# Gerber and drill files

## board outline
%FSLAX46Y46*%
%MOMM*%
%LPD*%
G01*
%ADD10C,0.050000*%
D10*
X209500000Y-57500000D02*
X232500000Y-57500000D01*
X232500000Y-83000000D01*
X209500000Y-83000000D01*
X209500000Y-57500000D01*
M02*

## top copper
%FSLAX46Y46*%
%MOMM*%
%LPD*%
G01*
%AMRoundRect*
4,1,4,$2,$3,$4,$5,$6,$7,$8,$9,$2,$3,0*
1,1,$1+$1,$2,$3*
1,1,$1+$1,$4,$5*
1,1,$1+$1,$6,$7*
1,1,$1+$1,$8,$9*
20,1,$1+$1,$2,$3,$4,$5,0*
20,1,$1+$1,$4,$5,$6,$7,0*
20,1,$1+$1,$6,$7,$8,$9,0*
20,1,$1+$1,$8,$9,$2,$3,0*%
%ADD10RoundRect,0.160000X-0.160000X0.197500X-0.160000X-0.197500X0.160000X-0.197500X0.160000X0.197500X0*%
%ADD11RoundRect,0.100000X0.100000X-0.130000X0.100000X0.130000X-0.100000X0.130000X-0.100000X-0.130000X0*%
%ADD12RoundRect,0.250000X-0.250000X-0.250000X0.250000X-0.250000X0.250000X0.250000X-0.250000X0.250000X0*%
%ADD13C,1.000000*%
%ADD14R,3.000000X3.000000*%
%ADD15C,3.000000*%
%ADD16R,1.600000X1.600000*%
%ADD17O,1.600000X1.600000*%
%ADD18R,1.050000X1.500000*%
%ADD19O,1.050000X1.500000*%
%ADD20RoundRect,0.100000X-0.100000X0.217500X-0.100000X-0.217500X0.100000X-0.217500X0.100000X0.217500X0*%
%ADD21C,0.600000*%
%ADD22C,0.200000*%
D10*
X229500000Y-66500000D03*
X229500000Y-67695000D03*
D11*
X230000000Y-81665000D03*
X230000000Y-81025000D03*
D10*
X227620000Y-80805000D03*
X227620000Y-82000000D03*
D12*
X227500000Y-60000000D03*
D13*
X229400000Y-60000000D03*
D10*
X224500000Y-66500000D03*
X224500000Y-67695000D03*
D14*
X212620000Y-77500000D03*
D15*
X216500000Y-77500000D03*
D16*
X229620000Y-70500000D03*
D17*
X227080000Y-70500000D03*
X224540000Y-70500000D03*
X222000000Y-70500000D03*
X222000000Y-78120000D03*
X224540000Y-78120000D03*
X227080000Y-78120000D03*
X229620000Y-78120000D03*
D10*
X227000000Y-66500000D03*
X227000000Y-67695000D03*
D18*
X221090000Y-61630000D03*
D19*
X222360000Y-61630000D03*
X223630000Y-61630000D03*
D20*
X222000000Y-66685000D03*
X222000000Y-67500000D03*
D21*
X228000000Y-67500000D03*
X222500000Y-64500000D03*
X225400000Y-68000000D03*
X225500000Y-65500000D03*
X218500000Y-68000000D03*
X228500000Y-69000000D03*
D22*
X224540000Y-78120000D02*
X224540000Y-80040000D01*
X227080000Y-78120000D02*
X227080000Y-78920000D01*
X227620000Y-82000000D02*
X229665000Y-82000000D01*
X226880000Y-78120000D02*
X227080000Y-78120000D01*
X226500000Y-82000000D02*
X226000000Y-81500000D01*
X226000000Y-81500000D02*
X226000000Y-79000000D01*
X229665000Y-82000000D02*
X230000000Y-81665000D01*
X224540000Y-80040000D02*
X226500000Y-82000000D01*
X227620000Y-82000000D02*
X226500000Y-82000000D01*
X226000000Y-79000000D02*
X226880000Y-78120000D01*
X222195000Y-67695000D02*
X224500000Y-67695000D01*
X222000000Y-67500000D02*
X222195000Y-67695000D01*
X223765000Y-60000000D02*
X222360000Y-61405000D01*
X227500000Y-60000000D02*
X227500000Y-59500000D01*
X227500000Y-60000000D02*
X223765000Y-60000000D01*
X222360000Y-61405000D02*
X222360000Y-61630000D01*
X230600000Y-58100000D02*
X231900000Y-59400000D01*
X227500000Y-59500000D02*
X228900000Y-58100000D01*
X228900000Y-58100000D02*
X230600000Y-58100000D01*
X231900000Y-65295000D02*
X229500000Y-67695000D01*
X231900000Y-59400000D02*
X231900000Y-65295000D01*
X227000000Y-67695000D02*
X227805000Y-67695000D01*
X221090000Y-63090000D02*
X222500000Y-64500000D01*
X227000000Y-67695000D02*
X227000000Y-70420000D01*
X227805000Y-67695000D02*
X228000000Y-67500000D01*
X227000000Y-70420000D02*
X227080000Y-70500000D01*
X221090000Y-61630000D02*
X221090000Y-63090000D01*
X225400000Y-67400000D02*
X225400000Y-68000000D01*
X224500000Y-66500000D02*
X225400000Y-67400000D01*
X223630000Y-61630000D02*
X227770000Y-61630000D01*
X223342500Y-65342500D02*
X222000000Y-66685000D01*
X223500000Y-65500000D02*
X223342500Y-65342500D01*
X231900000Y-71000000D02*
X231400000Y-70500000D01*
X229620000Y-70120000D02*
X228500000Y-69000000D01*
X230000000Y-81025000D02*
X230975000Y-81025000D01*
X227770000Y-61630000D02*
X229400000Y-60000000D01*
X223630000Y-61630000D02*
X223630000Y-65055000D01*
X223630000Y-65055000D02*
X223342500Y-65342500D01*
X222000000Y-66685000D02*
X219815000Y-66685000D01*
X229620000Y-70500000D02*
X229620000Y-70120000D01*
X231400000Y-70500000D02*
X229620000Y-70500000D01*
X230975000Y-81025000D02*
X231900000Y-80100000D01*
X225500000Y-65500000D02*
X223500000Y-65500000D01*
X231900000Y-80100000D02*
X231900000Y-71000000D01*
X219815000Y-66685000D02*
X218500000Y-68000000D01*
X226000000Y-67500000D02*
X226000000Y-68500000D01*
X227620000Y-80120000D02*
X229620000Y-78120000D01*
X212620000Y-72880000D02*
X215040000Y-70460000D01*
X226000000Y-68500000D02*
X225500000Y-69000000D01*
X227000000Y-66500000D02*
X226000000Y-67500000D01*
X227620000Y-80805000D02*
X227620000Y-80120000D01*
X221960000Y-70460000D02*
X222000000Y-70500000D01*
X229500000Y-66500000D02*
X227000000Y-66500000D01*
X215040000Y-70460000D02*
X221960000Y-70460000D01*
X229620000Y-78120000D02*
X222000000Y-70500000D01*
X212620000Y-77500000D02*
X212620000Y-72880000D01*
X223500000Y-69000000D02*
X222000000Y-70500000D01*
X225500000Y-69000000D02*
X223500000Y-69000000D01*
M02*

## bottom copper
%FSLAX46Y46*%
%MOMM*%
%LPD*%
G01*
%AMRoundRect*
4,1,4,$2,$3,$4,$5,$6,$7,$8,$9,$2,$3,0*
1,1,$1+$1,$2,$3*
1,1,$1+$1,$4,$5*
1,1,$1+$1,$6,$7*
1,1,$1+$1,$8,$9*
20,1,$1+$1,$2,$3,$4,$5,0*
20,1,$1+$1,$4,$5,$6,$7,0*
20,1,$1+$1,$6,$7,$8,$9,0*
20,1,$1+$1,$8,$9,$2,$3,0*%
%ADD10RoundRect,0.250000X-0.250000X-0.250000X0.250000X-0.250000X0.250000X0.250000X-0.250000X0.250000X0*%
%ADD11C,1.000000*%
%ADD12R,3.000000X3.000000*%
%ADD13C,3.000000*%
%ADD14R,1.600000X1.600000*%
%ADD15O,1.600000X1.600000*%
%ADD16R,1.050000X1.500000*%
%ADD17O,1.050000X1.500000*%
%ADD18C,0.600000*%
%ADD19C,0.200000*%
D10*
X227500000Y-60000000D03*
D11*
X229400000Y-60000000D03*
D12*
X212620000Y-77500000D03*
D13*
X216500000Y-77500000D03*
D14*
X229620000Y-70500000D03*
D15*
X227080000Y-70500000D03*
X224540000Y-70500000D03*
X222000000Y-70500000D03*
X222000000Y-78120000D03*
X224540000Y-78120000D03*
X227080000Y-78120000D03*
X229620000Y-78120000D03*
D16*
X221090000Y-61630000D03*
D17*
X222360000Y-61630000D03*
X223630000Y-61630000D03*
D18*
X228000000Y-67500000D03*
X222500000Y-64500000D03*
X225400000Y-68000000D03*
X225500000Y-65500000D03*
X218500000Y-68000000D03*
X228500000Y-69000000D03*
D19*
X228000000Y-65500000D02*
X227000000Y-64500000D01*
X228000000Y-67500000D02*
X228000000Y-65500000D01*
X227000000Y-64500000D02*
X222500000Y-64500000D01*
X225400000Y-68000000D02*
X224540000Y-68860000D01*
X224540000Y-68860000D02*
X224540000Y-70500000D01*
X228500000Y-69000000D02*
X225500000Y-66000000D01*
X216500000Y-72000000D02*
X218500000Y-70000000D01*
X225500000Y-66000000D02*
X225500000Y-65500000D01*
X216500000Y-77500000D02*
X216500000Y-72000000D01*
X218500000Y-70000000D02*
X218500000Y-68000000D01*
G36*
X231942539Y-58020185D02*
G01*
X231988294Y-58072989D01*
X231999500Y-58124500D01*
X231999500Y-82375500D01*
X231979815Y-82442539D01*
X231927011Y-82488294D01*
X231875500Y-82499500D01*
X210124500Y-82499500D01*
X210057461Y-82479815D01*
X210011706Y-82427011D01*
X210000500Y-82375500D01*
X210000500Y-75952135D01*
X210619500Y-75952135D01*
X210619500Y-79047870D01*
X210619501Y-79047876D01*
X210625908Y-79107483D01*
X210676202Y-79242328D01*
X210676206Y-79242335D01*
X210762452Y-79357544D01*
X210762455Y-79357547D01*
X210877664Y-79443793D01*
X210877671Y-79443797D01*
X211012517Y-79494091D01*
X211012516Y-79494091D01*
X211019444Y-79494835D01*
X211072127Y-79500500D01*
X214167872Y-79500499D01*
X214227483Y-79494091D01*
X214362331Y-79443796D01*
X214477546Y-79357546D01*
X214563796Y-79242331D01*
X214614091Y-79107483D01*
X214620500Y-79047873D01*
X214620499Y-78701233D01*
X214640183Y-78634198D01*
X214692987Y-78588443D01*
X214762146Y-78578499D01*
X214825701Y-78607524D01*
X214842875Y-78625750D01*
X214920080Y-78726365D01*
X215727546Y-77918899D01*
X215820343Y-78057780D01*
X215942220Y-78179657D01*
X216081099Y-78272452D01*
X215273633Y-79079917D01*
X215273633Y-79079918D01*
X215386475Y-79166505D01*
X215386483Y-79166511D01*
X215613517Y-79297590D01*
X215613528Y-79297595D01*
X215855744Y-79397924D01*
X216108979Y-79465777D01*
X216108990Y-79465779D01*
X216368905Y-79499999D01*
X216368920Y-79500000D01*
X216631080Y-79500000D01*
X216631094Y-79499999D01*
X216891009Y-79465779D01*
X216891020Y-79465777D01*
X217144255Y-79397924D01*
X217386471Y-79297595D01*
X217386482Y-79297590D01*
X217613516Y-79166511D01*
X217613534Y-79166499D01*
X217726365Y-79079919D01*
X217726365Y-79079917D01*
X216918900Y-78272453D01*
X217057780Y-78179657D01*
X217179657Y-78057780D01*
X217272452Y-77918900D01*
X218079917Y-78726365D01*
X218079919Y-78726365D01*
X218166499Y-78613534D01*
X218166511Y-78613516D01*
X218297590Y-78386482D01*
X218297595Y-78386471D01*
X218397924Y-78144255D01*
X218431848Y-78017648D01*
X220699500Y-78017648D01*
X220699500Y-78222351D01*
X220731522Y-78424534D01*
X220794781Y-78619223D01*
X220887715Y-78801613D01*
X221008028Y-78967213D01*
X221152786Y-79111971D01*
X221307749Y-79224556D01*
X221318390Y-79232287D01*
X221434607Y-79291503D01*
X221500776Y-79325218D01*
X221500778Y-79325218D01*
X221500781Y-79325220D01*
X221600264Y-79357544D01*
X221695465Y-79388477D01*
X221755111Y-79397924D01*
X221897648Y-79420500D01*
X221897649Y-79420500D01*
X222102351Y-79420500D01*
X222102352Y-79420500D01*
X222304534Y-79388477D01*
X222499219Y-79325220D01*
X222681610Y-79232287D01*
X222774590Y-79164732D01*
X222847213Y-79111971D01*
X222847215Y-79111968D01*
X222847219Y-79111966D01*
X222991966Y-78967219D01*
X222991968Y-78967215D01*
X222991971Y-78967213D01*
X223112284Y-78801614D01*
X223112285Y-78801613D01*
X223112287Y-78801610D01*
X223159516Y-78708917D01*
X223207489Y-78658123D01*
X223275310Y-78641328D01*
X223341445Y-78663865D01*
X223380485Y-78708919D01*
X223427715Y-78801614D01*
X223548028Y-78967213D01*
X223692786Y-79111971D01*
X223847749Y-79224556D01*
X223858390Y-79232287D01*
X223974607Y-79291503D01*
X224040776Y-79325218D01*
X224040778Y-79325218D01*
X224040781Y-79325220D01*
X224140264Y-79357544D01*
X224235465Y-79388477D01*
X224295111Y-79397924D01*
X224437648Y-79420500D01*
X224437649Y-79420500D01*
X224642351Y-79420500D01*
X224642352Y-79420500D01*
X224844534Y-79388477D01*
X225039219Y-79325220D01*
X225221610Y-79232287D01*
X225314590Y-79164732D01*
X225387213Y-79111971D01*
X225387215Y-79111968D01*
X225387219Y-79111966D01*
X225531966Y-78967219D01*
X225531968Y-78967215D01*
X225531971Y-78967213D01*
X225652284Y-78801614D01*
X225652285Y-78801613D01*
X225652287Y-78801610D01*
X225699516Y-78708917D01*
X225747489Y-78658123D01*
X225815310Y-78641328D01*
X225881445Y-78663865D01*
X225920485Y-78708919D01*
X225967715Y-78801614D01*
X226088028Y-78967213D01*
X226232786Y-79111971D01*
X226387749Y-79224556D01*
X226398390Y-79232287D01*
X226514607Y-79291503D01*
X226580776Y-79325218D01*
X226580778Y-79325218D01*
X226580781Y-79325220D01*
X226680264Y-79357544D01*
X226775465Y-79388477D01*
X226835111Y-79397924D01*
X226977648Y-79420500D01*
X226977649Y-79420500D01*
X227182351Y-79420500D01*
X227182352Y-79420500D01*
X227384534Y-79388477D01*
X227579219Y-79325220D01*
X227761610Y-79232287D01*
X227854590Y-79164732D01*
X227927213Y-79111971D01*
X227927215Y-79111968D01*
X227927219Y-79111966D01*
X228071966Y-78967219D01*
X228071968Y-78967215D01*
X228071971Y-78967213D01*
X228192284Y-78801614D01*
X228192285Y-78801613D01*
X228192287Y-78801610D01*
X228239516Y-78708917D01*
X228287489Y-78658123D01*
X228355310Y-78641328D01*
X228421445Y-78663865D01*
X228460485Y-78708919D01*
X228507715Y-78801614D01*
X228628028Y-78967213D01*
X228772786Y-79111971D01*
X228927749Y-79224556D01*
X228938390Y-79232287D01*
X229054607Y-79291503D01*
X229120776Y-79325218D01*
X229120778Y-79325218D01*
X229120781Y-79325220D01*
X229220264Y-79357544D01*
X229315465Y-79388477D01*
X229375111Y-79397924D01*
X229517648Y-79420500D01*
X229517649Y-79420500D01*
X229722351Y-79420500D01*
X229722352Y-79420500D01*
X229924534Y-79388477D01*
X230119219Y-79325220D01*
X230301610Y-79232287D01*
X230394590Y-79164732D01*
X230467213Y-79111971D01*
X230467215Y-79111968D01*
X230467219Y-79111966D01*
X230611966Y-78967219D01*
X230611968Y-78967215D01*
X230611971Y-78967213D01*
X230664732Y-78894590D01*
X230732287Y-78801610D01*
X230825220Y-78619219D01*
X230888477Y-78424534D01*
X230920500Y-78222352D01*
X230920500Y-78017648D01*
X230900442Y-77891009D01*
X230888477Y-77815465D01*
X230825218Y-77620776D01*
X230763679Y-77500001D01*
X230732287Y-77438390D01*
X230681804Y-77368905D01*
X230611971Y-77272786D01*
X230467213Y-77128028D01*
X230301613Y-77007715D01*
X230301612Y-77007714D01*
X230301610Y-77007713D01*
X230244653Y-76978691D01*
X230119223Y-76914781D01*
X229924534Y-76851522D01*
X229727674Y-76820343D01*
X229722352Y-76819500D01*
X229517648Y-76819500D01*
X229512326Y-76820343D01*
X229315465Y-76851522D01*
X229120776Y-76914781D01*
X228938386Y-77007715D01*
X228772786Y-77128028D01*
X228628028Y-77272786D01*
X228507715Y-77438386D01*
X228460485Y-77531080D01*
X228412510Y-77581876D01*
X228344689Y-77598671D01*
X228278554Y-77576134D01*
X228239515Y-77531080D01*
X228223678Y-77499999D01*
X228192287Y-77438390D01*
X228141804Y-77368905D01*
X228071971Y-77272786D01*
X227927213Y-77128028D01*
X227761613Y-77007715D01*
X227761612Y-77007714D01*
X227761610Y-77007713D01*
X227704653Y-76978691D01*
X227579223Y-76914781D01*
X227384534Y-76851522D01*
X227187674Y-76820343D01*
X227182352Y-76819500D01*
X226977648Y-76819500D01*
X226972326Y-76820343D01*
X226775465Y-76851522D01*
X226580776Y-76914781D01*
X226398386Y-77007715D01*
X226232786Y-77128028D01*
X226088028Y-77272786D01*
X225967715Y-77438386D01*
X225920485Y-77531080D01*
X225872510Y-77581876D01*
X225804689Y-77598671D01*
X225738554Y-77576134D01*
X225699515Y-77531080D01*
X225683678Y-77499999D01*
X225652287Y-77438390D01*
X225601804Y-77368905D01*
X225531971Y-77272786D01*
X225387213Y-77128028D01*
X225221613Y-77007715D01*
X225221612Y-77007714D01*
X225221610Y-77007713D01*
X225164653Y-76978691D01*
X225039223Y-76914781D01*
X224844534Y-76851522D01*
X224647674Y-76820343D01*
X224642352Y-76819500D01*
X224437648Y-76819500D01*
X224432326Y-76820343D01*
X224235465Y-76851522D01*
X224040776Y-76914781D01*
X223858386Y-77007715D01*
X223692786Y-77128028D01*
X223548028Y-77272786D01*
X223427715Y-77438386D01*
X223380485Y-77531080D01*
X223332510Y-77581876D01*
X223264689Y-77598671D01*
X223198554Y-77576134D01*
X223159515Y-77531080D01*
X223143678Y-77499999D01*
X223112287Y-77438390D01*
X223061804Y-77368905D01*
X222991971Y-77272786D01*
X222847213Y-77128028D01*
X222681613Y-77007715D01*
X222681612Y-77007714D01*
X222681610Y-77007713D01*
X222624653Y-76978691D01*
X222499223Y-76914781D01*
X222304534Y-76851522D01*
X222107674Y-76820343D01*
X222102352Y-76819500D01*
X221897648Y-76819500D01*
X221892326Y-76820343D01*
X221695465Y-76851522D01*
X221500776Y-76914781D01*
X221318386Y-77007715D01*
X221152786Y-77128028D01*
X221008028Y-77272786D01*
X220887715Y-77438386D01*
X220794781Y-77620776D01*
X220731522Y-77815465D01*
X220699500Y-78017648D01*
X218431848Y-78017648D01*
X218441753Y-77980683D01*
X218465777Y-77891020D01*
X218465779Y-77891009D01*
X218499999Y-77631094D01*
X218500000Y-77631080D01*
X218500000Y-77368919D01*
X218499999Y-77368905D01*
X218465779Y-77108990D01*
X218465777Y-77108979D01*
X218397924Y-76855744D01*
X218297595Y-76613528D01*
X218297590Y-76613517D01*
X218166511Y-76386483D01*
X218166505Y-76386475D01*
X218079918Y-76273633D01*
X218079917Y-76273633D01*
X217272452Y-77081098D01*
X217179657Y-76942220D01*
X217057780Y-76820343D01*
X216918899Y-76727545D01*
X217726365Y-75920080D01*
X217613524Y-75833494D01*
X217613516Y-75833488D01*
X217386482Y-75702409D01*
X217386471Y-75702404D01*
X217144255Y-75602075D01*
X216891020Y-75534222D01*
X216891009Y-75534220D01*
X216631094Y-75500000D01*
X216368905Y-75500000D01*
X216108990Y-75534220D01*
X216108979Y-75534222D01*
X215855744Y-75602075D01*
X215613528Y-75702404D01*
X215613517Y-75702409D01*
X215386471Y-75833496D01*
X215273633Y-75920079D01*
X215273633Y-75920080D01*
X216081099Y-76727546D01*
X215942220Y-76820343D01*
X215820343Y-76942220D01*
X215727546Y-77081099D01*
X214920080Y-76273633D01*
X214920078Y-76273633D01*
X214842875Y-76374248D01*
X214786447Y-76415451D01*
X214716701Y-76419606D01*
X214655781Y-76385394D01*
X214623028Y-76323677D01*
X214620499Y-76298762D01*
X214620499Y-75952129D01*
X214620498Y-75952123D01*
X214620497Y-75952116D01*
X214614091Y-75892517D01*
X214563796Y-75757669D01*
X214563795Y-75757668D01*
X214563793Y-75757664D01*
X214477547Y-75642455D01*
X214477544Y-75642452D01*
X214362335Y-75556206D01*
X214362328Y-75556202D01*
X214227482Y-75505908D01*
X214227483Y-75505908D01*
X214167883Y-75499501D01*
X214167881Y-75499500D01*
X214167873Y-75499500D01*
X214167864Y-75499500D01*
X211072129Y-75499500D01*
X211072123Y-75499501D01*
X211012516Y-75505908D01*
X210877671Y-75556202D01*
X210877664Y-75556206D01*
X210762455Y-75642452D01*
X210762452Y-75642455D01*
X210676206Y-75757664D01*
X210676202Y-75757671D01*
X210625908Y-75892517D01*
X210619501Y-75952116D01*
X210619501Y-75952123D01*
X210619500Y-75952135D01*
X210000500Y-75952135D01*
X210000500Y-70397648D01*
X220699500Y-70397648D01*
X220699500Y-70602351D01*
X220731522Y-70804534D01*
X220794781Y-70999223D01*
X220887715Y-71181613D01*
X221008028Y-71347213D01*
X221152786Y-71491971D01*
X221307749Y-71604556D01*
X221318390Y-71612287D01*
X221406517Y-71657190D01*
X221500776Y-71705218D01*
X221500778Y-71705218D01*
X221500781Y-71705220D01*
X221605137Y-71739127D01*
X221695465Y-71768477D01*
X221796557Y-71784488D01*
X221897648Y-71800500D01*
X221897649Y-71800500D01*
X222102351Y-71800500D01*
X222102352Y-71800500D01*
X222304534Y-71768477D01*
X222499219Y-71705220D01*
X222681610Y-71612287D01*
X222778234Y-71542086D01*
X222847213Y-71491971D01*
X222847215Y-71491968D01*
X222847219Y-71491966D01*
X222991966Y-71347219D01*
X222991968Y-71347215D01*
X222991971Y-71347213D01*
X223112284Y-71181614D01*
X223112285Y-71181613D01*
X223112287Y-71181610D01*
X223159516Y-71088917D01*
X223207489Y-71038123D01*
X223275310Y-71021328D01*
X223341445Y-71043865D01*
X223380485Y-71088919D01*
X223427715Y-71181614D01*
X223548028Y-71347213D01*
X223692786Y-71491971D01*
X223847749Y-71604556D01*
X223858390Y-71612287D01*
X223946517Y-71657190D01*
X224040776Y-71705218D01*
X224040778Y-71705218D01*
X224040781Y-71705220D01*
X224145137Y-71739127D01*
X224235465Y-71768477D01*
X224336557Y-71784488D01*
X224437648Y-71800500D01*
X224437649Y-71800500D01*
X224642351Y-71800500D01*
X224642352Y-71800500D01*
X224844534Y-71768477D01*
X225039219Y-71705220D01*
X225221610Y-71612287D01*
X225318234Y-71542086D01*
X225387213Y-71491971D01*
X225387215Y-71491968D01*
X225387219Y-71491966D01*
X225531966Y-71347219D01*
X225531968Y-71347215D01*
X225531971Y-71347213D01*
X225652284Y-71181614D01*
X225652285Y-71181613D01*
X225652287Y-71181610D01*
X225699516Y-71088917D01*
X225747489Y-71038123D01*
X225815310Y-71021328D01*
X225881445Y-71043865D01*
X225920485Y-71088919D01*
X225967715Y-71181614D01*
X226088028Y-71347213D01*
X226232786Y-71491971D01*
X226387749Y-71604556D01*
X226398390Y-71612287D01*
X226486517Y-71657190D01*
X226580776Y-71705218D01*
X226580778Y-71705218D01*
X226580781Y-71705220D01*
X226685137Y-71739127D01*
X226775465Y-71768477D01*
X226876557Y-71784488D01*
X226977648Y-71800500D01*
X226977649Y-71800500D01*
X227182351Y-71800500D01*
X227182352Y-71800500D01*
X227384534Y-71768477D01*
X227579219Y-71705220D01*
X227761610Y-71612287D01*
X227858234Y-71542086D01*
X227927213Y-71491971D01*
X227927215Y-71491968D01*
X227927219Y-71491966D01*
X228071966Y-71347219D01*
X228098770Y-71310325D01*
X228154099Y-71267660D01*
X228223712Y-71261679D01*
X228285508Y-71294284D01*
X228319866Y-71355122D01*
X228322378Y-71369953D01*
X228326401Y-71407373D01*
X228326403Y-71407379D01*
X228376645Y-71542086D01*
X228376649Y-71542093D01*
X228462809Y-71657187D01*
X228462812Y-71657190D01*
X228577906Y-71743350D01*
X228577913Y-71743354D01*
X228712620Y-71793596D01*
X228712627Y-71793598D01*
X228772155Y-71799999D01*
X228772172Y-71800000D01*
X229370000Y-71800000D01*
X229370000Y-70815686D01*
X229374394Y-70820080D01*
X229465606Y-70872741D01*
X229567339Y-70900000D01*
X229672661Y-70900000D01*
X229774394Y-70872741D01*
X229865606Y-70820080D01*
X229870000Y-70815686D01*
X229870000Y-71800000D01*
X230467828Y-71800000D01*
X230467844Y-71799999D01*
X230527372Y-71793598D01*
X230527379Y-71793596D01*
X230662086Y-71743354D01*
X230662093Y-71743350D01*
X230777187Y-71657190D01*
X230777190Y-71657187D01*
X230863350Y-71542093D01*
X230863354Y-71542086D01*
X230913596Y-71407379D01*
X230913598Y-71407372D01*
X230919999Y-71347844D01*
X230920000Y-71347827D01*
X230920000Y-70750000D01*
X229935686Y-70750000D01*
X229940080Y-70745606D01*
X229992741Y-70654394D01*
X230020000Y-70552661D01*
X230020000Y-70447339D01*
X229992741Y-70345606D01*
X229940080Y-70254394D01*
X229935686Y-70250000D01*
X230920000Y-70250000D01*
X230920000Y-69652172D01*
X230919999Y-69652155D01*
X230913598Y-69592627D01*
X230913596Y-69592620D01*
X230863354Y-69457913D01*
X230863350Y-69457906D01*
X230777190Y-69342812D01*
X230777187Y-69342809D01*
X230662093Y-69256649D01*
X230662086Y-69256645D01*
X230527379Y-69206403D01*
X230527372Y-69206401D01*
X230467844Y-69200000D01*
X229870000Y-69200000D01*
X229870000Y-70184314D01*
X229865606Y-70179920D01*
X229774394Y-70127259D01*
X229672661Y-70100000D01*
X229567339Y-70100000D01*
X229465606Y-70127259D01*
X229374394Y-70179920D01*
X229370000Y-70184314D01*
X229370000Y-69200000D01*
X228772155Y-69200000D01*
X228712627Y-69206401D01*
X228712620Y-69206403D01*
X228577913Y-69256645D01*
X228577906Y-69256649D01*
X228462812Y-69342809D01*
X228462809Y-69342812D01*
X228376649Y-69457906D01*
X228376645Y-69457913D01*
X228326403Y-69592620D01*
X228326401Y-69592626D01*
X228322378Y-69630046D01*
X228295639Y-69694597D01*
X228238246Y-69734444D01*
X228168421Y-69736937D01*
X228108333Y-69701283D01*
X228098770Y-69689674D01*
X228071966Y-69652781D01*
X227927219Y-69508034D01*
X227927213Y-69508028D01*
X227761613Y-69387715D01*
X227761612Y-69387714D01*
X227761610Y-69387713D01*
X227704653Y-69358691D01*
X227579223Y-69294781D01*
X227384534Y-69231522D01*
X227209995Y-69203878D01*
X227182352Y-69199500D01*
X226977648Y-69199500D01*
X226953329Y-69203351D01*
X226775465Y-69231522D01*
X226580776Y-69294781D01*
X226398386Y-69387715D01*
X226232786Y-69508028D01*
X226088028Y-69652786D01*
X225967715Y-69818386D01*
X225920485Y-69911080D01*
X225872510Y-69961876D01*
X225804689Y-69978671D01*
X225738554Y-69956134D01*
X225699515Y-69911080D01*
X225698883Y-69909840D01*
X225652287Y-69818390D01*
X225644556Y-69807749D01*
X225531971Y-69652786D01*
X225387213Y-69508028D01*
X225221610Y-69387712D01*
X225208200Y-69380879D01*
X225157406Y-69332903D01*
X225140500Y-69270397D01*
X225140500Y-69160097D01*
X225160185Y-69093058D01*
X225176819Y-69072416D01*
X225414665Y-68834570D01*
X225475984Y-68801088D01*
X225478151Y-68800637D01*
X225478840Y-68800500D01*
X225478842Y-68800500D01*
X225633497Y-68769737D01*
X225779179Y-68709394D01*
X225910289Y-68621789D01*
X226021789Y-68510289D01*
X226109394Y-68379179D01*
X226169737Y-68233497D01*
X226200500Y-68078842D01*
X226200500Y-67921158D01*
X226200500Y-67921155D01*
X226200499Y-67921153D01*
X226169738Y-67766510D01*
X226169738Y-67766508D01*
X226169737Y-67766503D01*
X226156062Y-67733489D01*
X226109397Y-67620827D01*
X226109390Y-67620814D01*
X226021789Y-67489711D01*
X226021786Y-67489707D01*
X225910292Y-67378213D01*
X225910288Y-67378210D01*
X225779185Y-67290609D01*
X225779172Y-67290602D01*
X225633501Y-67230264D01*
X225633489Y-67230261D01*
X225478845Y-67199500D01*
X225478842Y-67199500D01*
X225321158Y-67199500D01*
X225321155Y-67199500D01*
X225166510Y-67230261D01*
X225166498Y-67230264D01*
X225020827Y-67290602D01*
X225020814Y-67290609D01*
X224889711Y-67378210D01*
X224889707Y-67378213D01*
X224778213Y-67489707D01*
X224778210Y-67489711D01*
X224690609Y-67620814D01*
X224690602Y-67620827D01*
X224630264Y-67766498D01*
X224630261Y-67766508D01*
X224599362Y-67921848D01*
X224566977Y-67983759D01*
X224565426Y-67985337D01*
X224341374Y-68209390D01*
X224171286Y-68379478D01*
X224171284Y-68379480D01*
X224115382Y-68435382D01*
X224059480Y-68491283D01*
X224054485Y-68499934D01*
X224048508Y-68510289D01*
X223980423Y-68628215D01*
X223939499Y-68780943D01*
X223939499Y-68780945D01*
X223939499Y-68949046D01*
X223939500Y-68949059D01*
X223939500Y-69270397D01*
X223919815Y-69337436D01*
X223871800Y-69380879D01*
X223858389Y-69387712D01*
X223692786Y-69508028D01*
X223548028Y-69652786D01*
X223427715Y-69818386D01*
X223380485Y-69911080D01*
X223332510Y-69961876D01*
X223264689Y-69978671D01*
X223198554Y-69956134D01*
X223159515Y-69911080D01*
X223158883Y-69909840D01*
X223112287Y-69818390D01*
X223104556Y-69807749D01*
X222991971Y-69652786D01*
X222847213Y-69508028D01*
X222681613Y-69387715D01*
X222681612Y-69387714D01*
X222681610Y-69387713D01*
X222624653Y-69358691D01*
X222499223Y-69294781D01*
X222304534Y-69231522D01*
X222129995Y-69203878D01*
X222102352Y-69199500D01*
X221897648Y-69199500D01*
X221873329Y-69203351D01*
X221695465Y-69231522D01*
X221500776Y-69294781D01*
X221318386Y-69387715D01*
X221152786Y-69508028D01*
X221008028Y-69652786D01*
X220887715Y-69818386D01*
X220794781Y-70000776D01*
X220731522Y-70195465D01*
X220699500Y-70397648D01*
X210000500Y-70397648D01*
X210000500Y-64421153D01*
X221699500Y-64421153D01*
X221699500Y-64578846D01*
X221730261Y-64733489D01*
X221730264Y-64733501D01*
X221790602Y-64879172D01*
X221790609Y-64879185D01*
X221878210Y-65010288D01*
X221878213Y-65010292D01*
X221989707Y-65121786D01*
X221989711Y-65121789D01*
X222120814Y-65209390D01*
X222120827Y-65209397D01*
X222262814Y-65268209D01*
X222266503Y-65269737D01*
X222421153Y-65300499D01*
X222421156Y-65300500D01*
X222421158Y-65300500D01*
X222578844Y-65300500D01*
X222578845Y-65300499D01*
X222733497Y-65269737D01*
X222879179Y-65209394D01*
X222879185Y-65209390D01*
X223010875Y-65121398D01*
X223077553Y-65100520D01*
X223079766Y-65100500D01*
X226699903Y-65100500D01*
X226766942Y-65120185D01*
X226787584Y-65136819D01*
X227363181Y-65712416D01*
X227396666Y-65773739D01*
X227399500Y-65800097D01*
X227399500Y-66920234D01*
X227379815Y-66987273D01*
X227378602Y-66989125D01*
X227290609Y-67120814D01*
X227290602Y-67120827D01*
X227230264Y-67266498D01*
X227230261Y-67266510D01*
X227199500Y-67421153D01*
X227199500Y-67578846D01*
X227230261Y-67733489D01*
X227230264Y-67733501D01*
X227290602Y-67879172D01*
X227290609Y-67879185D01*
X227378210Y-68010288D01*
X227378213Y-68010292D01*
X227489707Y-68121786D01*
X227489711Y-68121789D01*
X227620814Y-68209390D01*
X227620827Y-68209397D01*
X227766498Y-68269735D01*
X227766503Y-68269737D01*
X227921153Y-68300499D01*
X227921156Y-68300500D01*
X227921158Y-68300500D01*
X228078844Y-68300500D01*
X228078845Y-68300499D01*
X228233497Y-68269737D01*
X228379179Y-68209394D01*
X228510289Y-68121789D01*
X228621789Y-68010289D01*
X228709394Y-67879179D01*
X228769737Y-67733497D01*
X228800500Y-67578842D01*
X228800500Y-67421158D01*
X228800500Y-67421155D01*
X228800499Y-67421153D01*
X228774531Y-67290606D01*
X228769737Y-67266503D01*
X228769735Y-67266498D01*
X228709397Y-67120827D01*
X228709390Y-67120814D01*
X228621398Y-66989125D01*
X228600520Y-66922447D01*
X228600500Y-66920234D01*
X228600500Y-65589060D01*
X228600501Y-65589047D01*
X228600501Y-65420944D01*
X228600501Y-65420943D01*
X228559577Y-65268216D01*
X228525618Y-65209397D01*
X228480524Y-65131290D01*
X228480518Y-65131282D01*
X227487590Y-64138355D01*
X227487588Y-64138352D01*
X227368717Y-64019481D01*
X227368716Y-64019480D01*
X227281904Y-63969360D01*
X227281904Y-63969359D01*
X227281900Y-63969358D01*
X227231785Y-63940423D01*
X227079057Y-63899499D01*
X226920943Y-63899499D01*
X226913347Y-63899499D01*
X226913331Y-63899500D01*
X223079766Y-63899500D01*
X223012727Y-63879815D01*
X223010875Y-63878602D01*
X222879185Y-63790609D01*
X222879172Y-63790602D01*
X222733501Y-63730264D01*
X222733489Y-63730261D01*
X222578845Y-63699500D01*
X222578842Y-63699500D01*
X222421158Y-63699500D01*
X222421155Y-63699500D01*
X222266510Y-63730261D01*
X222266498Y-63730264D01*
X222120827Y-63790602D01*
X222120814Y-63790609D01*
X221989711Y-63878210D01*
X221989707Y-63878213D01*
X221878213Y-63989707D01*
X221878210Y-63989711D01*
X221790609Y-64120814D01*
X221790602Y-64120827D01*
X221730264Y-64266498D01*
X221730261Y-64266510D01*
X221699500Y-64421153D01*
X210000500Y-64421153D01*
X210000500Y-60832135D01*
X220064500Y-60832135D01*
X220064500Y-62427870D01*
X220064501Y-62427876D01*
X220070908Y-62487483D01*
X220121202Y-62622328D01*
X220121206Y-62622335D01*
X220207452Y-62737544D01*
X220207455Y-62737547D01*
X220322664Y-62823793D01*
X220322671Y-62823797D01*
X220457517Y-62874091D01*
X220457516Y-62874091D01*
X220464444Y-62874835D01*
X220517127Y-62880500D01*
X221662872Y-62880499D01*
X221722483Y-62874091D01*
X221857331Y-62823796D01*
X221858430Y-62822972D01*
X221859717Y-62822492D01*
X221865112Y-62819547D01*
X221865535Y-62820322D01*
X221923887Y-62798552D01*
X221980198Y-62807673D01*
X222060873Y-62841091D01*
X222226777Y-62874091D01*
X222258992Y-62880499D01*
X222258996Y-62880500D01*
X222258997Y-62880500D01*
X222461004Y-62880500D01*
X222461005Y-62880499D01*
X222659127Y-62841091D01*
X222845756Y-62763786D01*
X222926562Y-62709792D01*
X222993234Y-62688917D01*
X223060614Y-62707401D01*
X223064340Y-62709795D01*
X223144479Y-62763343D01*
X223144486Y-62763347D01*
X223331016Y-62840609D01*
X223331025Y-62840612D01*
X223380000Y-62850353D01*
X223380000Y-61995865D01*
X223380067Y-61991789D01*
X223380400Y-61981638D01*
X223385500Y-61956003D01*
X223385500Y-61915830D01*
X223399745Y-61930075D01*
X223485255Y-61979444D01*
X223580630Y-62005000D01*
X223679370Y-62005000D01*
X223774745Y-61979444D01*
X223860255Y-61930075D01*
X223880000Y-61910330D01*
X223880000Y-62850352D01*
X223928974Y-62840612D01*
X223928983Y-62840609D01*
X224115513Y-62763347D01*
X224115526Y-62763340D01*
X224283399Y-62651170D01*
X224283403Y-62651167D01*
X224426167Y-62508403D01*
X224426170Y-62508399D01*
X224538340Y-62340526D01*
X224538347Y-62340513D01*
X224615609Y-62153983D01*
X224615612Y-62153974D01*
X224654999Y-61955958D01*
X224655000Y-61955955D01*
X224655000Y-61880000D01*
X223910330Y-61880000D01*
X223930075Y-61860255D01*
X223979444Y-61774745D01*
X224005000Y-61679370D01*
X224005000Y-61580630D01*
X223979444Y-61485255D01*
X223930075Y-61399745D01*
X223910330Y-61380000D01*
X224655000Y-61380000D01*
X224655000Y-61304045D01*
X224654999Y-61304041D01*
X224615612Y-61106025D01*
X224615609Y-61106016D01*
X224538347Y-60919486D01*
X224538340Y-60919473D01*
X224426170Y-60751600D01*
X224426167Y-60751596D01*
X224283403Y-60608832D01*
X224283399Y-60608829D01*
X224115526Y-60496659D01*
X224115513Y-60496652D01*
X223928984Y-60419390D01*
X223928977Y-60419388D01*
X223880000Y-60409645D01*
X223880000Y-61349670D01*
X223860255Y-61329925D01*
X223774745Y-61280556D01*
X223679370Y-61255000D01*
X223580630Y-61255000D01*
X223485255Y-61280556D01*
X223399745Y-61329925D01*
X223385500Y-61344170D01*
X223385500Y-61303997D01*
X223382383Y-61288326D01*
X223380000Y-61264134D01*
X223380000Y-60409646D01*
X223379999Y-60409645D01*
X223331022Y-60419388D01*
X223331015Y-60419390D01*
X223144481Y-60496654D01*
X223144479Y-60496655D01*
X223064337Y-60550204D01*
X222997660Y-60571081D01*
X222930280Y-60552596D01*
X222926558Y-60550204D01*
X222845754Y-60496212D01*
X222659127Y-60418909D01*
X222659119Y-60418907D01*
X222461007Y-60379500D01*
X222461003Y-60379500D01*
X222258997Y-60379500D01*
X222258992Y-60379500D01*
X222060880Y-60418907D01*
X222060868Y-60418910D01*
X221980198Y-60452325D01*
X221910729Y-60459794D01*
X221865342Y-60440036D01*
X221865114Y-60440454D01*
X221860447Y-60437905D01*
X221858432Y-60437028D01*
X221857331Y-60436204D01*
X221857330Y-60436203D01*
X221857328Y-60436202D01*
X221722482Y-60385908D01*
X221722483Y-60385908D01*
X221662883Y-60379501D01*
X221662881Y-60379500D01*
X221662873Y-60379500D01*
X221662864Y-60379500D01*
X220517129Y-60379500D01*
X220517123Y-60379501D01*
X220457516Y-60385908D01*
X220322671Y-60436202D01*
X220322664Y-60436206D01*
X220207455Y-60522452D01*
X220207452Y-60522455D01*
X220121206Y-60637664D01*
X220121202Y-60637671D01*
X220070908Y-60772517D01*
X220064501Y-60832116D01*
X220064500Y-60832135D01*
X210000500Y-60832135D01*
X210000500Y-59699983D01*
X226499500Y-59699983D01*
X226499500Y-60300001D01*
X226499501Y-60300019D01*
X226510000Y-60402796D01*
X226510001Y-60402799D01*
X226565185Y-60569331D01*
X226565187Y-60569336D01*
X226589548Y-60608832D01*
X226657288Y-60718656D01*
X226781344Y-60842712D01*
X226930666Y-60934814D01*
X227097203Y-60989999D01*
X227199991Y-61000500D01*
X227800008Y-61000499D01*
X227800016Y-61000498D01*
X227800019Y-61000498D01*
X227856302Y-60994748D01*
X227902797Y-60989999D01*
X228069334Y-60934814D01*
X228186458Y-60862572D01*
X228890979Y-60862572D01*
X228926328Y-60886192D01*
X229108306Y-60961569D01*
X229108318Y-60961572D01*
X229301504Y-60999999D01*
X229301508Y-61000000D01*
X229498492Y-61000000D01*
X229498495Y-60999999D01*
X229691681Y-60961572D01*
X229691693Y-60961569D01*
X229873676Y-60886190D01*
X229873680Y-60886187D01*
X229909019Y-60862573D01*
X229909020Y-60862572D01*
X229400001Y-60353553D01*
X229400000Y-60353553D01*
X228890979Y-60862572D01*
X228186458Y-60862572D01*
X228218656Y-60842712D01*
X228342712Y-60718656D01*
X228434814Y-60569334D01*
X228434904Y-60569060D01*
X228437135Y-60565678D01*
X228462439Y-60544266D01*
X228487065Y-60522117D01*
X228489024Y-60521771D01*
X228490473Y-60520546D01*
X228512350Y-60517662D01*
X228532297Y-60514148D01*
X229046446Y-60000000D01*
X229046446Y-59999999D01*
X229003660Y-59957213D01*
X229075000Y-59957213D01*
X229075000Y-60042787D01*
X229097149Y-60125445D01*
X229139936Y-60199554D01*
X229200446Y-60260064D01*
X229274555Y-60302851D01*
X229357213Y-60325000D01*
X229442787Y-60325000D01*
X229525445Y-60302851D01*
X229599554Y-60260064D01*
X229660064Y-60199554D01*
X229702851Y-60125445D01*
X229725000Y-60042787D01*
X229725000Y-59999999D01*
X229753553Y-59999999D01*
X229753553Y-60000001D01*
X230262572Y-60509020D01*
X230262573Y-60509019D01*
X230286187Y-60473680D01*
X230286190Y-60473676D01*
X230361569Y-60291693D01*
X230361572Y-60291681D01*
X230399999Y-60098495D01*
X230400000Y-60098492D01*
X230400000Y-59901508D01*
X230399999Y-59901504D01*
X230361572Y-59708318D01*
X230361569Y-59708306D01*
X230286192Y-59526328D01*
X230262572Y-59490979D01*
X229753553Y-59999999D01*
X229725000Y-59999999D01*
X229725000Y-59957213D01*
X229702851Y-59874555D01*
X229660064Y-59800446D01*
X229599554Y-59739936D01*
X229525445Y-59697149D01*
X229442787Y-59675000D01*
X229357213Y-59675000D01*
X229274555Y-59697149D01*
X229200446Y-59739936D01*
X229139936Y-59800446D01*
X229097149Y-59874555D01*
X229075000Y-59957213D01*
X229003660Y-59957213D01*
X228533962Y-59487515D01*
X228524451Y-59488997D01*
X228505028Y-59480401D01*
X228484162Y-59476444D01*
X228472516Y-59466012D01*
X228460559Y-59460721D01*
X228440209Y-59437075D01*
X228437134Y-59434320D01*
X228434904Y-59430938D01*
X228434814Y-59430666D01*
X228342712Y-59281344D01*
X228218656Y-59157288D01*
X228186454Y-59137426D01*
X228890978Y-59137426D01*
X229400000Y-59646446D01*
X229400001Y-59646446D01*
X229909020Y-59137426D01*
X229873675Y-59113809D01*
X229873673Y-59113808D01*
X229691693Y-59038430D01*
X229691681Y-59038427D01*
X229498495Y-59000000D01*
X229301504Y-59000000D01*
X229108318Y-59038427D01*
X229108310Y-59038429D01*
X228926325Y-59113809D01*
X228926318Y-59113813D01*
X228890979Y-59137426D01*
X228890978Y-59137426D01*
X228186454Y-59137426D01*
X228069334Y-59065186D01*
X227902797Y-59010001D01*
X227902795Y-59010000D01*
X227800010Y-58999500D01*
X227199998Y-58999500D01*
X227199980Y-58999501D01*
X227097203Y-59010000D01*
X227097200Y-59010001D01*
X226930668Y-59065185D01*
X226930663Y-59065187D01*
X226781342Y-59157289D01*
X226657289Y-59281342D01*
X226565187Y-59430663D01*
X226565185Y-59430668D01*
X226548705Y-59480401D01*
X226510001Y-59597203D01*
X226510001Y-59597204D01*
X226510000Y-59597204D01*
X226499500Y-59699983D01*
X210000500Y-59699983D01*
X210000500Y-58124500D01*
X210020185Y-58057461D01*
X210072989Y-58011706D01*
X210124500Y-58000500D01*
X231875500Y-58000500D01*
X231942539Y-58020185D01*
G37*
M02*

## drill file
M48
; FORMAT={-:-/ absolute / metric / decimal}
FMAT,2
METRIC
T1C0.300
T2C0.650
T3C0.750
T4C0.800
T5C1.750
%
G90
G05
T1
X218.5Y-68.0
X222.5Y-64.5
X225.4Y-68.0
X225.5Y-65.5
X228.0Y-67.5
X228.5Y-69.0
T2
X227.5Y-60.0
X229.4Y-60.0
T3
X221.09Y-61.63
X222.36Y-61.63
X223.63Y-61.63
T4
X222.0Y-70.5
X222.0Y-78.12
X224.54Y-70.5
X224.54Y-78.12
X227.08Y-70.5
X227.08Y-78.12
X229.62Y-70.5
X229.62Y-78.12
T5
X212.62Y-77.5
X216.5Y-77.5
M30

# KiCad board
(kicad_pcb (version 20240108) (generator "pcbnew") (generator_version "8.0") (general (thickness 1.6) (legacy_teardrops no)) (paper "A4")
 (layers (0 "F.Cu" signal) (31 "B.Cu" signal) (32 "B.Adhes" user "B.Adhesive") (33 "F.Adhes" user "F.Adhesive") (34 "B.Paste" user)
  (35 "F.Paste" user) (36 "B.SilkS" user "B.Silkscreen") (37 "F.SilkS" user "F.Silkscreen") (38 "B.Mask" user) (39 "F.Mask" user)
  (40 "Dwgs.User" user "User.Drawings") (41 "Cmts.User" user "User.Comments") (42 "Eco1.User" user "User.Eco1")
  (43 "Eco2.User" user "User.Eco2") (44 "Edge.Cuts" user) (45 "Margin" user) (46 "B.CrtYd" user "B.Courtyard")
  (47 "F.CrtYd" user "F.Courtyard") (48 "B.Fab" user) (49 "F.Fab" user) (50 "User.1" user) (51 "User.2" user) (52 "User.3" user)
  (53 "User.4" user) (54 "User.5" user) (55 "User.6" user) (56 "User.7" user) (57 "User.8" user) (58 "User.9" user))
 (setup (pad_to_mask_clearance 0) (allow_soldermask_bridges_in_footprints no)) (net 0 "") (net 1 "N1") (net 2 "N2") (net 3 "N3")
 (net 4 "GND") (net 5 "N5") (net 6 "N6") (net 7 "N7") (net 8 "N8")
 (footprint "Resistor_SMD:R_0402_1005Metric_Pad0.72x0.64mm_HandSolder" (layer "F.Cu") (at 229.5 67.0975 -90)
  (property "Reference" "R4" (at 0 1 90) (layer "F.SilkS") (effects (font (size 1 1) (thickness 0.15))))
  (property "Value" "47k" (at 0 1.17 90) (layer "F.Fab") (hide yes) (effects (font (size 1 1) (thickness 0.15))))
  (pad "1" smd roundrect (at -0.5975 0 270) (size 0.715 0.64) (layers "F.Cu" "F.Paste" "F.Mask") (roundrect_rratio 0.25) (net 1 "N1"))
  (pad "2" smd roundrect (at 0.5975 0 270) (size 0.715 0.64) (layers "F.Cu" "F.Paste" "F.Mask") (roundrect_rratio 0.25) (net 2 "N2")))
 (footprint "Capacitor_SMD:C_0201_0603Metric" (layer "F.Cu") (at 230 81.345 90)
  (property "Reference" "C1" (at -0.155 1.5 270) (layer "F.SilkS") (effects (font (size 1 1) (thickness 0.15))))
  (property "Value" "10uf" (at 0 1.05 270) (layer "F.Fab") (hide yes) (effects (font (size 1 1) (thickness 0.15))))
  (pad "" smd roundrect (at -0.345 0 90) (size 0.318 0.36) (layers "F.Paste") (roundrect_rratio 0.25))
  (pad "" smd roundrect (at 0.345 0 90) (size 0.318 0.36) (layers "F.Paste") (roundrect_rratio 0.25))
  (pad "1" smd roundrect (at -0.32 0 90) (size 0.46 0.4) (layers "F.Cu" "F.Mask") (roundrect_rratio 0.25) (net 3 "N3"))
  (pad "2" smd roundrect (at 0.32 0 90) (size 0.46 0.4) (layers "F.Cu" "F.Mask") (roundrect_rratio 0.25) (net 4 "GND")))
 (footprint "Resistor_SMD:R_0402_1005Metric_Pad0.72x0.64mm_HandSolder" (layer "F.Cu") (at 227.62 81.4025 -90)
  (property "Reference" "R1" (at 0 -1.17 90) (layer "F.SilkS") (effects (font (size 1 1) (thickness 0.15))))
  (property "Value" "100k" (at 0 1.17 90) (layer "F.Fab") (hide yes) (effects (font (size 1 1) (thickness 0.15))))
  (pad "1" smd roundrect (at -0.5975 0 270) (size 0.715 0.64) (layers "F.Cu" "F.Paste" "F.Mask") (roundrect_rratio 0.25) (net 1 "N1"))
  (pad "2" smd roundrect (at 0.5975 0 270) (size 0.715 0.64) (layers "F.Cu" "F.Paste" "F.Mask") (roundrect_rratio 0.25) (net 3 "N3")))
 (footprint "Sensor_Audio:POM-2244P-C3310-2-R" (layer "F.Cu") (at 227.5 60)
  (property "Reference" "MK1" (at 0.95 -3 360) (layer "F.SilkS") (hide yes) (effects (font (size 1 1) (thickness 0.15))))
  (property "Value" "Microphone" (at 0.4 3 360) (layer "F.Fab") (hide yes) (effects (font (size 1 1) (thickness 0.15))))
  (pad "1" thru_hole roundrect (at 0 0) (size 1 1) (drill 0.65) (layers "*.Cu" "*.Mask") (remove_unused_layers no) (roundrect_rratio 0.25)
   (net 2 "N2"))
  (pad "2" thru_hole circle (at 1.9 0) (size 1 1) (drill 0.65) (layers "*.Cu" "*.Mask") (remove_unused_layers no) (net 4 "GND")))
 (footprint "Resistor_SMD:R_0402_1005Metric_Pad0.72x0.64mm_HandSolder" (layer "F.Cu") (at 224.5 67.0975 -90)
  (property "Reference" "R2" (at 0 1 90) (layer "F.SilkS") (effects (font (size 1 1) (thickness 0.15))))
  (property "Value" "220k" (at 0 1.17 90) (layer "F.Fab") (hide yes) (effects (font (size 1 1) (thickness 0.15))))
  (pad "1" smd roundrect (at -0.5975 0 270) (size 0.715 0.64) (layers "F.Cu" "F.Paste" "F.Mask") (roundrect_rratio 0.25) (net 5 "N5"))
  (pad "2" smd roundrect (at 0.5975 0 270) (size 0.715 0.64) (layers "F.Cu" "F.Paste" "F.Mask") (roundrect_rratio 0.25) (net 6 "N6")))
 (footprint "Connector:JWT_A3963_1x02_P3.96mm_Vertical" (layer "F.Cu") (at 212.62 77.5)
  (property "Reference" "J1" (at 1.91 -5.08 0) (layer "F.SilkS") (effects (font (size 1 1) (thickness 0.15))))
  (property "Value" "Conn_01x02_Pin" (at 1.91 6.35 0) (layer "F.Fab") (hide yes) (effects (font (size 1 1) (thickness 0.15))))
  (pad "1" thru_hole rect (at 0 0) (size 3 3) (drill 1.75) (layers "*.Cu" "*.Mask") (remove_unused_layers no) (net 1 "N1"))
  (pad "2" thru_hole circle (at 3.88 0) (size 3 3) (drill 1.75) (layers "*.Cu" "*.Mask") (remove_unused_layers no) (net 4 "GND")))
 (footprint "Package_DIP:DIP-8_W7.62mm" (layer "F.Cu") (at 229.62 70.5 -90)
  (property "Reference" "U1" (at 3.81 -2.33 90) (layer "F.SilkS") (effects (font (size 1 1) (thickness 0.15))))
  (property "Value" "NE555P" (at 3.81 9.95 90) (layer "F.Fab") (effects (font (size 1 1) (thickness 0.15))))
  (pad "1" thru_hole rect (at 0 0 270) (size 1.6 1.6) (drill 0.8) (layers "*.Cu" "*.Mask") (remove_unused_layers no) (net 4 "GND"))
  (pad "2" thru_hole oval (at 0 2.54 270) (size 1.6 1.6) (drill 0.8) (layers "*.Cu" "*.Mask") (remove_unused_layers no) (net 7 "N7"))
  (pad "3" thru_hole oval (at 0 5.08 270) (size 1.6 1.6) (drill 0.8) (layers "*.Cu" "*.Mask") (remove_unused_layers no) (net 5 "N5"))
  (pad "4" thru_hole oval (at 0 7.62 270) (size 1.6 1.6) (drill 0.8) (layers "*.Cu" "*.Mask") (remove_unused_layers no) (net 1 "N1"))
  (pad "5" thru_hole oval (at 7.62 7.62 270) (size 1.6 1.6) (drill 0.8) (layers "*.Cu" "*.Mask") (remove_unused_layers no) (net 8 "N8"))
  (pad "6" thru_hole oval (at 7.62 5.08 270) (size 1.6 1.6) (drill 0.8) (layers "*.Cu" "*.Mask") (remove_unused_layers no) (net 3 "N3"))
  (pad "7" thru_hole oval (at 7.62 2.54 270) (size 1.6 1.6) (drill 0.8) (layers "*.Cu" "*.Mask") (remove_unused_layers no) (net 3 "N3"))
  (pad "8" thru_hole oval (at 7.62 0 270) (size 1.6 1.6) (drill 0.8) (layers "*.Cu" "*.Mask") (remove_unused_layers no) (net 1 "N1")))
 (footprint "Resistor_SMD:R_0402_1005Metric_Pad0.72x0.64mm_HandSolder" (layer "F.Cu") (at 227 67.0975 -90)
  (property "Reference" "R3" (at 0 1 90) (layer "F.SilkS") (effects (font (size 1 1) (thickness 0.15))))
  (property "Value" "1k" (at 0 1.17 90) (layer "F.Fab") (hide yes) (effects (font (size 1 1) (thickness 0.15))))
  (pad "1" smd roundrect (at -0.5975 0 270) (size 0.715 0.64) (layers "F.Cu" "F.Paste" "F.Mask") (roundrect_rratio 0.25) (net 1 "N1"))
  (pad "2" smd roundrect (at 0.5975 0 270) (size 0.715 0.64) (layers "F.Cu" "F.Paste" "F.Mask") (roundrect_rratio 0.25) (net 7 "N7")))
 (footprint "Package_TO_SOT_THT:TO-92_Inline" (layer "F.Cu") (at 221.09 61.63)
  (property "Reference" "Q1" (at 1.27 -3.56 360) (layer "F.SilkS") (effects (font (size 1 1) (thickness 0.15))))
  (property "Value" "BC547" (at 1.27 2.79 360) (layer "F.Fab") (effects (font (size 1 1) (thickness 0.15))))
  (pad "1" thru_hole rect (at 0 0) (size 1.05 1.5) (drill 0.75) (layers "*.Cu" "*.Mask") (remove_unused_layers no) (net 7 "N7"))
  (pad "2" thru_hole oval (at 1.27 0) (size 1.05 1.5) (drill 0.75) (layers "*.Cu" "*.Mask") (remove_unused_layers no) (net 2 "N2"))
  (pad "3" thru_hole oval (at 2.54 0) (size 1.05 1.5) (drill 0.75) (layers "*.Cu" "*.Mask") (remove_unused_layers no) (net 4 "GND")))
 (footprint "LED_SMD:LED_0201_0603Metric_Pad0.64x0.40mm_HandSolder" (layer "F.Cu") (at 222 67.0925 -90)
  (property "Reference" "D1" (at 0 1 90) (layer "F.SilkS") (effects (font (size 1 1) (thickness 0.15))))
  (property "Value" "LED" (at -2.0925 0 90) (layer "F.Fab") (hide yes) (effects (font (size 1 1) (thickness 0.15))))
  (pad "" smd roundrect (at -0.4325 0 270) (size 0.458 0.36) (layers "F.Paste") (roundrect_rratio 0.25))
  (pad "" smd roundrect (at 0.4325 0 270) (size 0.458 0.36) (layers "F.Paste") (roundrect_rratio 0.25))
  (pad "1" smd roundrect (at -0.4075 0 270) (size 0.635 0.4) (layers "F.Cu" "F.Mask") (roundrect_rratio 0.25) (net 4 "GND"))
  (pad "2" smd roundrect (at 0.4075 0 270) (size 0.635 0.4) (layers "F.Cu" "F.Mask") (roundrect_rratio 0.25) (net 6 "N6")))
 (gr_rect (start 209.5 57.5) (end 232.5 83) (stroke (width 0.05) (type default)) (fill none) (layer "Edge.Cuts"))
 (segment (start 224.54 78.12) (end 224.54 80.04) (width 0.2) (layer "F.Cu") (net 3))
 (segment (start 227.08 78.12) (end 227.08 78.92) (width 0.2) (layer "F.Cu") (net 3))
 (segment (start 227.62 82) (end 229.665 82) (width 0.2) (layer "F.Cu") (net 3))
 (segment (start 226.88 78.12) (end 227.08 78.12) (width 0.2) (layer "F.Cu") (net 3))
 (segment (start 226.5 82) (end 226 81.5) (width 0.2) (layer "F.Cu") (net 3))
 (segment (start 226 81.5) (end 226 79) (width 0.2) (layer "F.Cu") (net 3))
 (segment (start 229.665 82) (end 230 81.665) (width 0.2) (layer "F.Cu") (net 3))
 (segment (start 224.54 80.04) (end 226.5 82) (width 0.2) (layer "F.Cu") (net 3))
 (segment (start 227.62 82) (end 226.5 82) (width 0.2) (layer "F.Cu") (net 3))
 (segment (start 226 79) (end 226.88 78.12) (width 0.2) (layer "F.Cu") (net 3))
 (segment (start 222.195 67.695) (end 224.5 67.695) (width 0.2) (layer "F.Cu") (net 6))
 (segment (start 222 67.5) (end 222.195 67.695) (width 0.2) (layer "F.Cu") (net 6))
 (segment (start 223.765 60) (end 222.36 61.405) (width 0.2) (layer "F.Cu") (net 2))
 (segment (start 227.5 60) (end 227.5 59.5) (width 0.2) (layer "F.Cu") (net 2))
 (segment (start 227.5 60) (end 223.765 60) (width 0.2) (layer "F.Cu") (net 2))
 (segment (start 222.36 61.405) (end 222.36 61.63) (width 0.2) (layer "F.Cu") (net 2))
 (segment (start 230.6 58.1) (end 231.9 59.4) (width 0.2) (layer "F.Cu") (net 2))
 (segment (start 227.5 59.5) (end 228.9 58.1) (width 0.2) (layer "F.Cu") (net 2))
 (segment (start 228.9 58.1) (end 230.6 58.1) (width 0.2) (layer "F.Cu") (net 2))
 (segment (start 231.9 65.295) (end 229.5 67.695) (width 0.2) (layer "F.Cu") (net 2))
 (segment (start 231.9 59.4) (end 231.9 65.295) (width 0.2) (layer "F.Cu") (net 2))
 (segment (start 227 67.695) (end 227.805 67.695) (width 0.2) (layer "F.Cu") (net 7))
 (segment (start 221.09 63.09) (end 222.5 64.5) (width 0.2) (layer "F.Cu") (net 7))
 (segment (start 227 67.695) (end 227 70.42) (width 0.2) (layer "F.Cu") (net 7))
 (segment (start 227.805 67.695) (end 228 67.5) (width 0.2) (layer "F.Cu") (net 7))
 (segment (start 227 70.42) (end 227.08 70.5) (width 0.2) (layer "F.Cu") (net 7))
 (segment (start 221.09 61.63) (end 221.09 63.09) (width 0.2) (layer "F.Cu") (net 7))
 (via (at 228 67.5) (size 0.6) (drill 0.3) (layers "F.Cu" "B.Cu") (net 7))
 (via (at 222.5 64.5) (size 0.6) (drill 0.3) (layers "F.Cu" "B.Cu") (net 7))
 (segment (start 228 65.5) (end 227 64.5) (width 0.2) (layer "B.Cu") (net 7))
 (segment (start 228 67.5) (end 228 65.5) (width 0.2) (layer "B.Cu") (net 7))
 (segment (start 227 64.5) (end 222.5 64.5) (width 0.2) (layer "B.Cu") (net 7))
 (segment (start 225.4 67.4) (end 225.4 68) (width 0.2) (layer "F.Cu") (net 5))
 (segment (start 224.5 66.5) (end 225.4 67.4) (width 0.2) (layer "F.Cu") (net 5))
 (via (at 225.4 68) (size 0.6) (drill 0.3) (layers "F.Cu" "B.Cu") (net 5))
 (segment (start 225.4 68) (end 224.54 68.86) (width 0.2) (layer "B.Cu") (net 5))
 (segment (start 224.54 68.86) (end 224.54 70.5) (width 0.2) (layer "B.Cu") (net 5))
 (segment (start 223.63 61.63) (end 227.77 61.63) (width 0.2) (layer "F.Cu") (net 4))
 (segment (start 223.3425 65.3425) (end 222 66.685) (width 0.2) (layer "F.Cu") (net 4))
 (segment (start 223.5 65.5) (end 223.3425 65.3425) (width 0.2) (layer "F.Cu") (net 4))
 (segment (start 231.9 71) (end 231.4 70.5) (width 0.2) (layer "F.Cu") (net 4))
 (segment (start 229.62 70.12) (end 228.5 69) (width 0.2) (layer "F.Cu") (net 4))
 (segment (start 230 81.025) (end 230.975 81.025) (width 0.2) (layer "F.Cu") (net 4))
 (segment (start 227.77 61.63) (end 229.4 60) (width 0.2) (layer "F.Cu") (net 4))
 (segment (start 223.63 61.63) (end 223.63 65.055) (width 0.2) (layer "F.Cu") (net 4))
 (segment (start 223.63 65.055) (end 223.3425 65.3425) (width 0.2) (layer "F.Cu") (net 4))
 (segment (start 222 66.685) (end 219.815 66.685) (width 0.2) (layer "F.Cu") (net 4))
 (segment (start 229.62 70.5) (end 229.62 70.12) (width 0.2) (layer "F.Cu") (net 4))
 (segment (start 231.4 70.5) (end 229.62 70.5) (width 0.2) (layer "F.Cu") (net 4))
 (segment (start 230.975 81.025) (end 231.9 80.1) (width 0.2) (layer "F.Cu") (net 4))
 (segment (start 225.5 65.5) (end 223.5 65.5) (width 0.2) (layer "F.Cu") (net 4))
 (segment (start 231.9 80.1) (end 231.9 71) (width 0.2) (layer "F.Cu") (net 4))
 (segment (start 219.815 66.685) (end 218.5 68) (width 0.2) (layer "F.Cu") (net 4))
 (via (at 225.5 65.5) (size 0.6) (drill 0.3) (layers "F.Cu" "B.Cu") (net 4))
 (via (at 218.5 68) (size 0.6) (drill 0.3) (layers "F.Cu" "B.Cu") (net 4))
 (via (at 228.5 69) (size 0.6) (drill 0.3) (layers "F.Cu" "B.Cu") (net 4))
 (segment (start 228.5 69) (end 225.5 66) (width 0.2) (layer "B.Cu") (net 4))
 (segment (start 216.5 72) (end 218.5 70) (width 0.2) (layer "B.Cu") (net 4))
 (segment (start 225.5 66) (end 225.5 65.5) (width 0.2) (layer "B.Cu") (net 4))
 (segment (start 216.5 77.5) (end 216.5 72) (width 0.2) (layer "B.Cu") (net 4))
 (segment (start 218.5 70) (end 218.5 68) (width 0.2) (layer "B.Cu") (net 4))
 (segment (start 226 67.5) (end 226 68.5) (width 0.2) (layer "F.Cu") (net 1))
 (segment (start 227.62 80.12) (end 229.62 78.12) (width 0.2) (layer "F.Cu") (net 1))
 (segment (start 212.62 72.88) (end 215.04 70.46) (width 0.2) (layer "F.Cu") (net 1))
 (segment (start 226 68.5) (end 225.5 69) (width 0.2) (layer "F.Cu") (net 1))
 (segment (start 227 66.5) (end 226 67.5) (width 0.2) (layer "F.Cu") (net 1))
 (segment (start 227.62 80.805) (end 227.62 80.12) (width 0.2) (layer "F.Cu") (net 1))
 (segment (start 221.96 70.46) (end 222 70.5) (width 0.2) (layer "F.Cu") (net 1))
 (segment (start 229.5 66.5) (end 227 66.5) (width 0.2) (layer "F.Cu") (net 1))
 (segment (start 215.04 70.46) (end 221.96 70.46) (width 0.2) (layer "F.Cu") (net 1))
 (segment (start 229.62 78.12) (end 222 70.5) (width 0.2) (layer "F.Cu") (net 1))
 (segment (start 212.62 77.5) (end 212.62 72.88) (width 0.2) (layer "F.Cu") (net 1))
 (segment (start 223.5 69) (end 222 70.5) (width 0.2) (layer "F.Cu") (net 1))
 (segment (start 225.5 69) (end 223.5 69) (width 0.2) (layer "F.Cu") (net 1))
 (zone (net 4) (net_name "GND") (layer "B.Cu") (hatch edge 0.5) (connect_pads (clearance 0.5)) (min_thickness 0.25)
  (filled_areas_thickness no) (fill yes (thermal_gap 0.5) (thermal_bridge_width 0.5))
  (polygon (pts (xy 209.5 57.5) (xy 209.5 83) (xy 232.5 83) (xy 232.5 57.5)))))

